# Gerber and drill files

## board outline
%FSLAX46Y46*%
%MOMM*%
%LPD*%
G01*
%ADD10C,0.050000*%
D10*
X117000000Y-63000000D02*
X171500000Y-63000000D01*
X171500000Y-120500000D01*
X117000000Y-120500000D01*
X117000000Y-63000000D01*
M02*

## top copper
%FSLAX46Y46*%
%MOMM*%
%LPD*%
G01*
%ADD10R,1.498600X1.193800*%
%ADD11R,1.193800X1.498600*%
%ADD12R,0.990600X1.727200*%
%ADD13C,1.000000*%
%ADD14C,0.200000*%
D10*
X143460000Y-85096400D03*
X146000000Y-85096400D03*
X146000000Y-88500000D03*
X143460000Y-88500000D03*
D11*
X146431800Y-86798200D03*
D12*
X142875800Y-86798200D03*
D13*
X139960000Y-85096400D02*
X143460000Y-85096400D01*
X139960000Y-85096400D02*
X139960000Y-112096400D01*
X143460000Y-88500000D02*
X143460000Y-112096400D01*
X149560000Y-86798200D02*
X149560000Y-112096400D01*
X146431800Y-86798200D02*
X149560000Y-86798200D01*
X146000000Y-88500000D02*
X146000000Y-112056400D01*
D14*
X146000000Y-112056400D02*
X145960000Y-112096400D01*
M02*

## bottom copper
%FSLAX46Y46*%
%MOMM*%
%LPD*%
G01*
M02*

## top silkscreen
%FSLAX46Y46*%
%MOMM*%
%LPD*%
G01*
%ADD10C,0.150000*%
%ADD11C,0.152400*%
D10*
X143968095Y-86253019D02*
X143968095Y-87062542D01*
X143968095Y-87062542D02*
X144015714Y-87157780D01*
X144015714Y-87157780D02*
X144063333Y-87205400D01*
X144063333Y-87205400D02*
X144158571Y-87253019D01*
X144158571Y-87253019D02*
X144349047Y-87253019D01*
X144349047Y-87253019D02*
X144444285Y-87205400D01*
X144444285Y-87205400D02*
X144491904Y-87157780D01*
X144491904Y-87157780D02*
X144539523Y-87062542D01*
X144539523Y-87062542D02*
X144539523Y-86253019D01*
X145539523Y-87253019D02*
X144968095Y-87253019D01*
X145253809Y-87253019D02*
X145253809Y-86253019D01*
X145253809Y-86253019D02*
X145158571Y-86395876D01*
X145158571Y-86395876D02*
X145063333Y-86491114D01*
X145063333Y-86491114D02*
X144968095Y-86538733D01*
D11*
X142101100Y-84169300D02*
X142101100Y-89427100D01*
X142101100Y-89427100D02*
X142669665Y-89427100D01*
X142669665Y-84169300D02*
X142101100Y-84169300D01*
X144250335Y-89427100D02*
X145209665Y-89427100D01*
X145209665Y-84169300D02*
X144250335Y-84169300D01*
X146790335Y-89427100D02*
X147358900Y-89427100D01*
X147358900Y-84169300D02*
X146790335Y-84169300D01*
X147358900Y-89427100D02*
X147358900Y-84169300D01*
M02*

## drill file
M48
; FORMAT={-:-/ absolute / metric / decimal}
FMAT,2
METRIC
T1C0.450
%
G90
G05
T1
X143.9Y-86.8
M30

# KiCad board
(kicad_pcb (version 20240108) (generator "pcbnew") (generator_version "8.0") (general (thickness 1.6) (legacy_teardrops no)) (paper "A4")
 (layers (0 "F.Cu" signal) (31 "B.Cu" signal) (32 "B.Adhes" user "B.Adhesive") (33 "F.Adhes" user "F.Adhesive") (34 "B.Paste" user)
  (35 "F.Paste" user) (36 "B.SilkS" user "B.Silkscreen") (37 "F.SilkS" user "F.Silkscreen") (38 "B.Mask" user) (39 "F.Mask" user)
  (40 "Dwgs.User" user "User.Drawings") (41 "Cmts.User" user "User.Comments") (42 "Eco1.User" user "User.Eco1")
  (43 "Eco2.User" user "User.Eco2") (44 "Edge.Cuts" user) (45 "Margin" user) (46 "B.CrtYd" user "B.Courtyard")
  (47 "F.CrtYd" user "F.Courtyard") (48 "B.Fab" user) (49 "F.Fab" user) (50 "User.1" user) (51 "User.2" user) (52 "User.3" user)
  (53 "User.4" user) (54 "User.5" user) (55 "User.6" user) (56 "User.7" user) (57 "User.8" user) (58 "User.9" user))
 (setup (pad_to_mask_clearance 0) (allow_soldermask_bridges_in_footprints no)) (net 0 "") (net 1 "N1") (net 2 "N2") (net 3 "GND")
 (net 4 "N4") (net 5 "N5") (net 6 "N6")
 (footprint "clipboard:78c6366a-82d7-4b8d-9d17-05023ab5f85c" (layer "F.Cu") (at 143.9 86.8)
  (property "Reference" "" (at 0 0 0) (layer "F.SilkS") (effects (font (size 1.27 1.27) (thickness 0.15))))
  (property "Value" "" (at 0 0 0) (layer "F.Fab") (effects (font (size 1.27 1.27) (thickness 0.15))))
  (pad "" np_thru_hole circle (at 0 0) (size 0.45 0.45) (drill 0.45) (layers "*.Mask")))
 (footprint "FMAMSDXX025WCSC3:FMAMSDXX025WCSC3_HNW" (layer "F.Cu") (at 144.73 86.7982)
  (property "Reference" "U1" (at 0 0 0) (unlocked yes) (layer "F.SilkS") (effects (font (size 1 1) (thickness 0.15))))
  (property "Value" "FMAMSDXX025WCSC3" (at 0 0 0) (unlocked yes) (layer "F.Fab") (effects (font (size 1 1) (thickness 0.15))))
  (fp_line (start -2.6289 -2.6289) (end -2.6289 2.6289) (stroke (width 0.1524) (type solid)) (layer "F.SilkS"))
  (fp_line (start -2.6289 2.6289) (end -2.060335 2.6289) (stroke (width 0.1524) (type solid)) (layer "F.SilkS"))
  (fp_line (start -2.060335 -2.6289) (end -2.6289 -2.6289) (stroke (width 0.1524) (type solid)) (layer "F.SilkS"))
  (fp_line (start -0.479665 2.6289) (end 0.479665 2.6289) (stroke (width 0.1524) (type solid)) (layer "F.SilkS"))
  (fp_line (start 0.479665 -2.6289) (end -0.479665 -2.6289) (stroke (width 0.1524) (type solid)) (layer "F.SilkS"))
  (fp_line (start 2.060335 2.6289) (end 2.6289 2.6289) (stroke (width 0.1524) (type solid)) (layer "F.SilkS"))
  (fp_line (start 2.6289 -2.6289) (end 2.060335 -2.6289) (stroke (width 0.1524) (type solid)) (layer "F.SilkS"))
  (fp_line (start 2.6289 2.6289) (end 2.6289 -2.6289) (stroke (width 0.1524) (type solid)) (layer "F.SilkS"))
  (pad "1" smd rect (at -1.27 -1.7018) (size 1.4986 1.1938) (layers "F.Cu" "F.Paste" "F.Mask") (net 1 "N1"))
  (pad "2" smd rect (at 1.27 -1.7018) (size 1.4986 1.1938) (layers "F.Cu" "F.Paste" "F.Mask") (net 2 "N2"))
  (pad "3" smd rect (at 1.27 1.7018) (size 1.4986 1.1938) (layers "F.Cu" "F.Paste" "F.Mask") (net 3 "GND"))
  (pad "4" smd rect (at -1.27 1.7018) (size 1.4986 1.1938) (layers "F.Cu" "F.Paste" "F.Mask") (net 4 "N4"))
  (pad "5" smd rect (at 1.7018 0) (size 1.1938 1.4986) (layers "F.Cu" "F.Mask") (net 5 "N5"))
  (pad "6" smd rect (at -1.8542 0) (size 0.9906 1.7272) (layers "F.Cu" "F.Paste" "F.Mask") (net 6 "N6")))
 (gr_rect (start 117 63) (end 171.5 120.5) (stroke (width 0.05) (type default)) (fill none) (layer "Edge.Cuts"))
 (segment (start 139.96 85.0964) (end 143.46 85.0964) (width 1) (layer "F.Cu") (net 1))
 (segment (start 139.96 85.0964) (end 139.96 112.0964) (width 1) (layer "F.Cu") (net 1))
 (segment (start 143.46 88.5) (end 143.46 112.0964) (width 1) (layer "F.Cu") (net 4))
 (segment (start 149.56 86.7982) (end 149.56 112.0964) (width 1) (layer "F.Cu") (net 5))
 (segment (start 146.4318 86.7982) (end 149.56 86.7982) (width 1) (layer "F.Cu") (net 5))
 (segment (start 146 88.5) (end 146 112.0564) (width 1) (layer "F.Cu") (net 3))
 (segment (start 146 112.0564) (end 145.96 112.0964) (width 0.2) (layer "F.Cu") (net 3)))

